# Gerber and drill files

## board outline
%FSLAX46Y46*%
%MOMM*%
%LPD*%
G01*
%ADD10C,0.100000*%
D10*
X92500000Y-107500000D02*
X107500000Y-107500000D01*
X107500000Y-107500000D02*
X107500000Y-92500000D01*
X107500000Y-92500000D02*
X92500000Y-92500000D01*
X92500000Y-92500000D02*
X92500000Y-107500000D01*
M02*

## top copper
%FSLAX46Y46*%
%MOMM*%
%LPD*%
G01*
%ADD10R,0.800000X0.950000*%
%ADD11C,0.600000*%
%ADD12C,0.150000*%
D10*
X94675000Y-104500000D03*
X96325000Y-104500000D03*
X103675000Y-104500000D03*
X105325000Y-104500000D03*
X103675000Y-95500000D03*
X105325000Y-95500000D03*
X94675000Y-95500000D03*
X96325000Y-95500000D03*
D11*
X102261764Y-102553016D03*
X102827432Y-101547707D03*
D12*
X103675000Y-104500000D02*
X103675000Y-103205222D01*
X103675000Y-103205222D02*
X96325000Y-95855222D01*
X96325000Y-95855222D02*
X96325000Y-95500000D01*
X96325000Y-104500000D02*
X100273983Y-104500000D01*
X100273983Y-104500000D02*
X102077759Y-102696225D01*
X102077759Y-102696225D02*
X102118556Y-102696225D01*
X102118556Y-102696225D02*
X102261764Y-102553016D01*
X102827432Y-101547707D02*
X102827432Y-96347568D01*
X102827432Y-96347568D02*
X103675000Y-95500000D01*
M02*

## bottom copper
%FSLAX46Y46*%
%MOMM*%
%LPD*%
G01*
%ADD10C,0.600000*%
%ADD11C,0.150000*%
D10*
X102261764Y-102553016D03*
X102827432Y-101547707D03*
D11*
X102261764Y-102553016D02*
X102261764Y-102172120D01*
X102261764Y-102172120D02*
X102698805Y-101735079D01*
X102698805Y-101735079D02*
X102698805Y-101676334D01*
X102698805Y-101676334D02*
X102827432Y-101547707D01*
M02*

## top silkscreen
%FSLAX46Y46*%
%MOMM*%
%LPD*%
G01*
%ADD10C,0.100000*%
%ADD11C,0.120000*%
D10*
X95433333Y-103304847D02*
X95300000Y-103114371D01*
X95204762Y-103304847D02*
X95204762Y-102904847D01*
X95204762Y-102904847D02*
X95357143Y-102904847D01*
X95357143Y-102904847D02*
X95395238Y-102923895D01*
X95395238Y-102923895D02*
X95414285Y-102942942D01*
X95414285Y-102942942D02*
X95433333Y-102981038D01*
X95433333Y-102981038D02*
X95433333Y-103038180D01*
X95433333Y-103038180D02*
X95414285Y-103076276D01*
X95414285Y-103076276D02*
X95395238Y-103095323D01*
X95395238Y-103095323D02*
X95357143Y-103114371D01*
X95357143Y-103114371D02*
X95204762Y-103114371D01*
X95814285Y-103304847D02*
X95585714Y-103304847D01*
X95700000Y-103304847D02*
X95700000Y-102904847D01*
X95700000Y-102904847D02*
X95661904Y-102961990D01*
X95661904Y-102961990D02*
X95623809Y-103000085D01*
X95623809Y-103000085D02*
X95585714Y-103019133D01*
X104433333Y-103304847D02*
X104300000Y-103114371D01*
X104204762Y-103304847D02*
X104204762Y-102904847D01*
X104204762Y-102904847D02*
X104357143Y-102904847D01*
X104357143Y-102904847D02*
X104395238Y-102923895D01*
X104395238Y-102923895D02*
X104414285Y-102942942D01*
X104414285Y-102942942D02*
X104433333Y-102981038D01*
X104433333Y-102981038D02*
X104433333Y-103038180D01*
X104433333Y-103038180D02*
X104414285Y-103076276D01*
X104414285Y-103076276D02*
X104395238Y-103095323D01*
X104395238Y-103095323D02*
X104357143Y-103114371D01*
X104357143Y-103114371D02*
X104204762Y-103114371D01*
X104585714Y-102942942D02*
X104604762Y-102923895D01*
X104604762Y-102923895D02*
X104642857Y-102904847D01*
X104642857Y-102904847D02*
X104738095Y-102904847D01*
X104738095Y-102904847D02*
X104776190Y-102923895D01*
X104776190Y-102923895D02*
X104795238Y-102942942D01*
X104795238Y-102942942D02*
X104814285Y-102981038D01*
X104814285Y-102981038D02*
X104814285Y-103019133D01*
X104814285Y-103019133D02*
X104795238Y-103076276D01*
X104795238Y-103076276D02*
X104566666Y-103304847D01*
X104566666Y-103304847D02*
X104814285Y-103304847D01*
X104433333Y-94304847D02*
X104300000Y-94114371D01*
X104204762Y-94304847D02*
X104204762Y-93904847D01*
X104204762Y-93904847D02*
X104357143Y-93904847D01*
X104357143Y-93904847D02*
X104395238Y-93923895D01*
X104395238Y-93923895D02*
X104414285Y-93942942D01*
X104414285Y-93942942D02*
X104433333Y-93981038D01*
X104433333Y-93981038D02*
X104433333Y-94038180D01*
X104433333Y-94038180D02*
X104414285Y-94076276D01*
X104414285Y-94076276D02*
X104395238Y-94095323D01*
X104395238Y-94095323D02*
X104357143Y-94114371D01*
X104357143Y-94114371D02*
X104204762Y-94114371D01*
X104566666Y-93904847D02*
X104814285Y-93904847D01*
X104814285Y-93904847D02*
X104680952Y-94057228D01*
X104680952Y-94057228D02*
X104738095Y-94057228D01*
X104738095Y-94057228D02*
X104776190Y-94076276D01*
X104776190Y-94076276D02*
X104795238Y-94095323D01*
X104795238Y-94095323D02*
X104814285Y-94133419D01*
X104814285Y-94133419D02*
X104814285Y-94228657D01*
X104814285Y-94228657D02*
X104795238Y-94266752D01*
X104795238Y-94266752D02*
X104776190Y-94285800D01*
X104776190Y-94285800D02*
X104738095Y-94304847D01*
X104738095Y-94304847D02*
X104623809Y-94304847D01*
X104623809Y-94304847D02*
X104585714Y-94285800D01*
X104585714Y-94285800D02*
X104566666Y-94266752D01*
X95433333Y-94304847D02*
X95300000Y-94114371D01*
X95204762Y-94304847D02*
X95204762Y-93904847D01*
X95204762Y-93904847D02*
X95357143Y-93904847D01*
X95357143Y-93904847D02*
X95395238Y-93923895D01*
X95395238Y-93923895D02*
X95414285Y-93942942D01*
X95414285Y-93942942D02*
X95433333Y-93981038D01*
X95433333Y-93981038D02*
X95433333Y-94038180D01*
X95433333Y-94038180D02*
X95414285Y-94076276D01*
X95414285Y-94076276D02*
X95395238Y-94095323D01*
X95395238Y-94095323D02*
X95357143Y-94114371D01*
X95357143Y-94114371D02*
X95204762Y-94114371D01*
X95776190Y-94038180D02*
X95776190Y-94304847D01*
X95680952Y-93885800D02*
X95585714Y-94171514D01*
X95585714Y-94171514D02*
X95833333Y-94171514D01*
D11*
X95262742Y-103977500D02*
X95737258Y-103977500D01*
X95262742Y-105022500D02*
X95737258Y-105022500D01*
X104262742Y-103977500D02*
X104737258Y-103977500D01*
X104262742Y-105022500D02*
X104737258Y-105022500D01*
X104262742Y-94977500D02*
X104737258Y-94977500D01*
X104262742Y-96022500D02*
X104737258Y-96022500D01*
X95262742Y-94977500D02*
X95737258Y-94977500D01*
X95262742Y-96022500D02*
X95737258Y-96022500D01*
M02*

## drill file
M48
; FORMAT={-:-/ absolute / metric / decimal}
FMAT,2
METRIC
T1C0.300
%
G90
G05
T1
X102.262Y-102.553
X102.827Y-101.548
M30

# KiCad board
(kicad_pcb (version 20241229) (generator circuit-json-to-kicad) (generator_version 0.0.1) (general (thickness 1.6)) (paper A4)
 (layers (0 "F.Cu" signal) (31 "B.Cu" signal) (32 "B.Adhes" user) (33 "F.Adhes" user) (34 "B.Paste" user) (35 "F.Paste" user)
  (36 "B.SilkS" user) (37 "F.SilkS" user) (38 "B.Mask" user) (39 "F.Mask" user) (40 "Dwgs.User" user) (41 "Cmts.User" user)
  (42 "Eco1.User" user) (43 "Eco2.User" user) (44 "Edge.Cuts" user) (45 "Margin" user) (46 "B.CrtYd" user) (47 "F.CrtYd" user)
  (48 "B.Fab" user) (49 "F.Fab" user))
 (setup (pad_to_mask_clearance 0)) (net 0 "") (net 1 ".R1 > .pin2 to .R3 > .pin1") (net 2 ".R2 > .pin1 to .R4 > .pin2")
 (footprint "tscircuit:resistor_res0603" (layer F.Cu) (at 95.5 104.5 0)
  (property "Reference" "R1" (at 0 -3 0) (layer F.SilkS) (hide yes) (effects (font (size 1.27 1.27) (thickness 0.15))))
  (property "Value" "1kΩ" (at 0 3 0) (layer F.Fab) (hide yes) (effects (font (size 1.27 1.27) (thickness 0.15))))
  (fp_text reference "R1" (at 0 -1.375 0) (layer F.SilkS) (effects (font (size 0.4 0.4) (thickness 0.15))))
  (fp_line (start -0.23725799999999975 -0.5225) (end 0.23725799999999975 -0.5225) (stroke (width 0.12) (type default)) (layer F.SilkS))
  (fp_line (start -0.23725799999999975 0.5225) (end 0.23725799999999975 0.5225) (stroke (width 0.12) (type default)) (layer F.SilkS))
  (pad "1" smd rect (at -0.8250000000000002 0 0) (size 0.8 0.95) (layers F.Cu F.Mask))
  (pad "2" smd rect (at 0.8250000000000002 0 0) (size 0.8 0.95) (layers F.Cu F.Mask) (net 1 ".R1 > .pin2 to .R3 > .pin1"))
  (pad "" smd rect (at -0.8250000000000002 0 0) (size 0.5599999999999999 0.6649999999999999) (layers F.Paste))
  (pad "" smd rect (at 0.8250000000000002 0 0) (size 0.5599999999999999 0.6649999999999999) (layers F.Paste)))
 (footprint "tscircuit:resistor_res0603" (layer F.Cu) (at 104.5 104.5 0)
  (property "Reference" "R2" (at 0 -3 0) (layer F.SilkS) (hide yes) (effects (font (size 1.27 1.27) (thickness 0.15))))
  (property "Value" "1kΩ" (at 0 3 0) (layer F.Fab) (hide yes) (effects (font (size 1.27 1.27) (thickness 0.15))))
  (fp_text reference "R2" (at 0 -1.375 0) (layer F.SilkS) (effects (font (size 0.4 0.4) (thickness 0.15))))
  (fp_line (start -0.23725799999999975 -0.5225) (end 0.23725799999999975 -0.5225) (stroke (width 0.12) (type default)) (layer F.SilkS))
  (fp_line (start -0.23725799999999975 0.5225) (end 0.23725799999999975 0.5225) (stroke (width 0.12) (type default)) (layer F.SilkS))
  (pad "1" smd rect (at -0.8250000000000002 0 0) (size 0.8 0.95) (layers F.Cu F.Mask) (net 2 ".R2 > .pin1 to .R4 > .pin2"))
  (pad "2" smd rect (at 0.8250000000000002 0 0) (size 0.8 0.95) (layers F.Cu F.Mask))
  (pad "" smd rect (at -0.8250000000000002 0 0) (size 0.5599999999999999 0.6649999999999999) (layers F.Paste))
  (pad "" smd rect (at 0.8250000000000002 0 0) (size 0.5599999999999999 0.6649999999999999) (layers F.Paste)))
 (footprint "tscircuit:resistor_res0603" (layer F.Cu) (at 104.5 95.5 0)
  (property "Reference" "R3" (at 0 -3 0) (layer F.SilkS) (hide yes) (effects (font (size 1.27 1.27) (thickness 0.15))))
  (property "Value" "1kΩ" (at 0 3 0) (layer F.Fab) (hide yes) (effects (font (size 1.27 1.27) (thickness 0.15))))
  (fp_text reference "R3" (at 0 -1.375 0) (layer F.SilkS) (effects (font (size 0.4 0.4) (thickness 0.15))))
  (fp_line (start -0.23725799999999975 -0.5225) (end 0.23725799999999975 -0.5225) (stroke (width 0.12) (type default)) (layer F.SilkS))
  (fp_line (start -0.23725799999999975 0.5225) (end 0.23725799999999975 0.5225) (stroke (width 0.12) (type default)) (layer F.SilkS))
  (pad "1" smd rect (at -0.8250000000000002 0 0) (size 0.8 0.95) (layers F.Cu F.Mask) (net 1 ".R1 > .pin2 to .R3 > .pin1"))
  (pad "2" smd rect (at 0.8250000000000002 0 0) (size 0.8 0.95) (layers F.Cu F.Mask))
  (pad "" smd rect (at -0.8250000000000002 0 0) (size 0.5599999999999999 0.6649999999999999) (layers F.Paste))
  (pad "" smd rect (at 0.8250000000000002 0 0) (size 0.5599999999999999 0.6649999999999999) (layers F.Paste)))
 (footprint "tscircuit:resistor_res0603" (layer F.Cu) (at 95.5 95.5 0)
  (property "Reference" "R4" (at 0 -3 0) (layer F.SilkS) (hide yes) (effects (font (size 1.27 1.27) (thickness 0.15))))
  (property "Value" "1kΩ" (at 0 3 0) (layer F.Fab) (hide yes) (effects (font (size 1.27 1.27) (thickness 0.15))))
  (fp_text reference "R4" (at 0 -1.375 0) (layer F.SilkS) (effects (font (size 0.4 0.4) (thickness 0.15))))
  (fp_line (start -0.23725799999999975 -0.5225) (end 0.23725799999999975 -0.5225) (stroke (width 0.12) (type default)) (layer F.SilkS))
  (fp_line (start -0.23725799999999975 0.5225) (end 0.23725799999999975 0.5225) (stroke (width 0.12) (type default)) (layer F.SilkS))
  (pad "1" smd rect (at -0.8250000000000002 0 0) (size 0.8 0.95) (layers F.Cu F.Mask))
  (pad "2" smd rect (at 0.8250000000000002 0 0) (size 0.8 0.95) (layers F.Cu F.Mask) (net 2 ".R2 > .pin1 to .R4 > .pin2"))
  (pad "" smd rect (at -0.8250000000000002 0 0) (size 0.5599999999999999 0.6649999999999999) (layers F.Paste))
  (pad "" smd rect (at 0.8250000000000002 0 0) (size 0.5599999999999999 0.6649999999999999) (layers F.Paste)))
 (segment (start 103.675 104.5) (end 103.675 103.20522221656093) (width 0.15) (layer F.Cu) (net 2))
 (segment (start 103.675 103.20522221656093) (end 96.325 95.85522221656093) (width 0.15) (layer F.Cu) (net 2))
 (segment (start 96.325 95.85522221656093) (end 96.325 95.5) (width 0.15) (layer F.Cu) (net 2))
 (segment (start 96.325 104.5) (end 100.27398336301454 104.5) (width 0.15) (layer F.Cu) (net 1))
 (segment (start 100.27398336301454 104.5) (end 102.07775883665545 102.6962245263591) (width 0.15) (layer F.Cu) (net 1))
 (segment (start 102.07775883665545 102.6962245263591) (end 102.11855550254027 102.6962245263591) (width 0.15) (layer F.Cu) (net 1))
 (segment (start 102.11855550254027 102.6962245263591) (end 102.26176395699403 102.55301607190533) (width 0.15) (layer F.Cu) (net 1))
 (segment (start 102.26176395699403 102.55301607190533) (end 102.26176395699403 102.17212026201244) (width 0.15) (layer B.Cu) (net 1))
 (segment (start 102.26176395699403 102.17212026201244) (end 102.69880482967297 101.7350793893335) (width 0.15) (layer B.Cu) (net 1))
 (segment (start 102.69880482967297 101.7350793893335) (end 102.69880482967297 101.67633448099376) (width 0.15) (layer B.Cu) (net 1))
 (segment (start 102.69880482967297 101.67633448099376) (end 102.82743246752361 101.54770684314312) (width 0.15) (layer B.Cu) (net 1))
 (segment (start 102.82743246752361 101.54770684314312) (end 102.82743246752361 96.34756753247639) (width 0.15) (layer F.Cu) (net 1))
 (segment (start 102.82743246752361 96.34756753247639) (end 103.675 95.5) (width 0.15) (layer F.Cu) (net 1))
 (gr_line (start 92.5 107.5) (end 107.5 107.5) (width 0.1) (layer Edge.Cuts))
 (gr_line (start 107.5 107.5) (end 107.5 92.5) (width 0.1) (layer Edge.Cuts))
 (gr_line (start 107.5 92.5) (end 92.5 92.5) (width 0.1) (layer Edge.Cuts))
 (gr_line (start 92.5 92.5) (end 92.5 107.5) (width 0.1) (layer Edge.Cuts))
 (via (at 102.26176395699403 102.55301607190533) (size 0.6) (drill 0.3) (layers F.Cu B.Cu) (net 1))
 (via (at 102.82743246752361 101.54770684314312) (size 0.6) (drill 0.3) (layers F.Cu B.Cu) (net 1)))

